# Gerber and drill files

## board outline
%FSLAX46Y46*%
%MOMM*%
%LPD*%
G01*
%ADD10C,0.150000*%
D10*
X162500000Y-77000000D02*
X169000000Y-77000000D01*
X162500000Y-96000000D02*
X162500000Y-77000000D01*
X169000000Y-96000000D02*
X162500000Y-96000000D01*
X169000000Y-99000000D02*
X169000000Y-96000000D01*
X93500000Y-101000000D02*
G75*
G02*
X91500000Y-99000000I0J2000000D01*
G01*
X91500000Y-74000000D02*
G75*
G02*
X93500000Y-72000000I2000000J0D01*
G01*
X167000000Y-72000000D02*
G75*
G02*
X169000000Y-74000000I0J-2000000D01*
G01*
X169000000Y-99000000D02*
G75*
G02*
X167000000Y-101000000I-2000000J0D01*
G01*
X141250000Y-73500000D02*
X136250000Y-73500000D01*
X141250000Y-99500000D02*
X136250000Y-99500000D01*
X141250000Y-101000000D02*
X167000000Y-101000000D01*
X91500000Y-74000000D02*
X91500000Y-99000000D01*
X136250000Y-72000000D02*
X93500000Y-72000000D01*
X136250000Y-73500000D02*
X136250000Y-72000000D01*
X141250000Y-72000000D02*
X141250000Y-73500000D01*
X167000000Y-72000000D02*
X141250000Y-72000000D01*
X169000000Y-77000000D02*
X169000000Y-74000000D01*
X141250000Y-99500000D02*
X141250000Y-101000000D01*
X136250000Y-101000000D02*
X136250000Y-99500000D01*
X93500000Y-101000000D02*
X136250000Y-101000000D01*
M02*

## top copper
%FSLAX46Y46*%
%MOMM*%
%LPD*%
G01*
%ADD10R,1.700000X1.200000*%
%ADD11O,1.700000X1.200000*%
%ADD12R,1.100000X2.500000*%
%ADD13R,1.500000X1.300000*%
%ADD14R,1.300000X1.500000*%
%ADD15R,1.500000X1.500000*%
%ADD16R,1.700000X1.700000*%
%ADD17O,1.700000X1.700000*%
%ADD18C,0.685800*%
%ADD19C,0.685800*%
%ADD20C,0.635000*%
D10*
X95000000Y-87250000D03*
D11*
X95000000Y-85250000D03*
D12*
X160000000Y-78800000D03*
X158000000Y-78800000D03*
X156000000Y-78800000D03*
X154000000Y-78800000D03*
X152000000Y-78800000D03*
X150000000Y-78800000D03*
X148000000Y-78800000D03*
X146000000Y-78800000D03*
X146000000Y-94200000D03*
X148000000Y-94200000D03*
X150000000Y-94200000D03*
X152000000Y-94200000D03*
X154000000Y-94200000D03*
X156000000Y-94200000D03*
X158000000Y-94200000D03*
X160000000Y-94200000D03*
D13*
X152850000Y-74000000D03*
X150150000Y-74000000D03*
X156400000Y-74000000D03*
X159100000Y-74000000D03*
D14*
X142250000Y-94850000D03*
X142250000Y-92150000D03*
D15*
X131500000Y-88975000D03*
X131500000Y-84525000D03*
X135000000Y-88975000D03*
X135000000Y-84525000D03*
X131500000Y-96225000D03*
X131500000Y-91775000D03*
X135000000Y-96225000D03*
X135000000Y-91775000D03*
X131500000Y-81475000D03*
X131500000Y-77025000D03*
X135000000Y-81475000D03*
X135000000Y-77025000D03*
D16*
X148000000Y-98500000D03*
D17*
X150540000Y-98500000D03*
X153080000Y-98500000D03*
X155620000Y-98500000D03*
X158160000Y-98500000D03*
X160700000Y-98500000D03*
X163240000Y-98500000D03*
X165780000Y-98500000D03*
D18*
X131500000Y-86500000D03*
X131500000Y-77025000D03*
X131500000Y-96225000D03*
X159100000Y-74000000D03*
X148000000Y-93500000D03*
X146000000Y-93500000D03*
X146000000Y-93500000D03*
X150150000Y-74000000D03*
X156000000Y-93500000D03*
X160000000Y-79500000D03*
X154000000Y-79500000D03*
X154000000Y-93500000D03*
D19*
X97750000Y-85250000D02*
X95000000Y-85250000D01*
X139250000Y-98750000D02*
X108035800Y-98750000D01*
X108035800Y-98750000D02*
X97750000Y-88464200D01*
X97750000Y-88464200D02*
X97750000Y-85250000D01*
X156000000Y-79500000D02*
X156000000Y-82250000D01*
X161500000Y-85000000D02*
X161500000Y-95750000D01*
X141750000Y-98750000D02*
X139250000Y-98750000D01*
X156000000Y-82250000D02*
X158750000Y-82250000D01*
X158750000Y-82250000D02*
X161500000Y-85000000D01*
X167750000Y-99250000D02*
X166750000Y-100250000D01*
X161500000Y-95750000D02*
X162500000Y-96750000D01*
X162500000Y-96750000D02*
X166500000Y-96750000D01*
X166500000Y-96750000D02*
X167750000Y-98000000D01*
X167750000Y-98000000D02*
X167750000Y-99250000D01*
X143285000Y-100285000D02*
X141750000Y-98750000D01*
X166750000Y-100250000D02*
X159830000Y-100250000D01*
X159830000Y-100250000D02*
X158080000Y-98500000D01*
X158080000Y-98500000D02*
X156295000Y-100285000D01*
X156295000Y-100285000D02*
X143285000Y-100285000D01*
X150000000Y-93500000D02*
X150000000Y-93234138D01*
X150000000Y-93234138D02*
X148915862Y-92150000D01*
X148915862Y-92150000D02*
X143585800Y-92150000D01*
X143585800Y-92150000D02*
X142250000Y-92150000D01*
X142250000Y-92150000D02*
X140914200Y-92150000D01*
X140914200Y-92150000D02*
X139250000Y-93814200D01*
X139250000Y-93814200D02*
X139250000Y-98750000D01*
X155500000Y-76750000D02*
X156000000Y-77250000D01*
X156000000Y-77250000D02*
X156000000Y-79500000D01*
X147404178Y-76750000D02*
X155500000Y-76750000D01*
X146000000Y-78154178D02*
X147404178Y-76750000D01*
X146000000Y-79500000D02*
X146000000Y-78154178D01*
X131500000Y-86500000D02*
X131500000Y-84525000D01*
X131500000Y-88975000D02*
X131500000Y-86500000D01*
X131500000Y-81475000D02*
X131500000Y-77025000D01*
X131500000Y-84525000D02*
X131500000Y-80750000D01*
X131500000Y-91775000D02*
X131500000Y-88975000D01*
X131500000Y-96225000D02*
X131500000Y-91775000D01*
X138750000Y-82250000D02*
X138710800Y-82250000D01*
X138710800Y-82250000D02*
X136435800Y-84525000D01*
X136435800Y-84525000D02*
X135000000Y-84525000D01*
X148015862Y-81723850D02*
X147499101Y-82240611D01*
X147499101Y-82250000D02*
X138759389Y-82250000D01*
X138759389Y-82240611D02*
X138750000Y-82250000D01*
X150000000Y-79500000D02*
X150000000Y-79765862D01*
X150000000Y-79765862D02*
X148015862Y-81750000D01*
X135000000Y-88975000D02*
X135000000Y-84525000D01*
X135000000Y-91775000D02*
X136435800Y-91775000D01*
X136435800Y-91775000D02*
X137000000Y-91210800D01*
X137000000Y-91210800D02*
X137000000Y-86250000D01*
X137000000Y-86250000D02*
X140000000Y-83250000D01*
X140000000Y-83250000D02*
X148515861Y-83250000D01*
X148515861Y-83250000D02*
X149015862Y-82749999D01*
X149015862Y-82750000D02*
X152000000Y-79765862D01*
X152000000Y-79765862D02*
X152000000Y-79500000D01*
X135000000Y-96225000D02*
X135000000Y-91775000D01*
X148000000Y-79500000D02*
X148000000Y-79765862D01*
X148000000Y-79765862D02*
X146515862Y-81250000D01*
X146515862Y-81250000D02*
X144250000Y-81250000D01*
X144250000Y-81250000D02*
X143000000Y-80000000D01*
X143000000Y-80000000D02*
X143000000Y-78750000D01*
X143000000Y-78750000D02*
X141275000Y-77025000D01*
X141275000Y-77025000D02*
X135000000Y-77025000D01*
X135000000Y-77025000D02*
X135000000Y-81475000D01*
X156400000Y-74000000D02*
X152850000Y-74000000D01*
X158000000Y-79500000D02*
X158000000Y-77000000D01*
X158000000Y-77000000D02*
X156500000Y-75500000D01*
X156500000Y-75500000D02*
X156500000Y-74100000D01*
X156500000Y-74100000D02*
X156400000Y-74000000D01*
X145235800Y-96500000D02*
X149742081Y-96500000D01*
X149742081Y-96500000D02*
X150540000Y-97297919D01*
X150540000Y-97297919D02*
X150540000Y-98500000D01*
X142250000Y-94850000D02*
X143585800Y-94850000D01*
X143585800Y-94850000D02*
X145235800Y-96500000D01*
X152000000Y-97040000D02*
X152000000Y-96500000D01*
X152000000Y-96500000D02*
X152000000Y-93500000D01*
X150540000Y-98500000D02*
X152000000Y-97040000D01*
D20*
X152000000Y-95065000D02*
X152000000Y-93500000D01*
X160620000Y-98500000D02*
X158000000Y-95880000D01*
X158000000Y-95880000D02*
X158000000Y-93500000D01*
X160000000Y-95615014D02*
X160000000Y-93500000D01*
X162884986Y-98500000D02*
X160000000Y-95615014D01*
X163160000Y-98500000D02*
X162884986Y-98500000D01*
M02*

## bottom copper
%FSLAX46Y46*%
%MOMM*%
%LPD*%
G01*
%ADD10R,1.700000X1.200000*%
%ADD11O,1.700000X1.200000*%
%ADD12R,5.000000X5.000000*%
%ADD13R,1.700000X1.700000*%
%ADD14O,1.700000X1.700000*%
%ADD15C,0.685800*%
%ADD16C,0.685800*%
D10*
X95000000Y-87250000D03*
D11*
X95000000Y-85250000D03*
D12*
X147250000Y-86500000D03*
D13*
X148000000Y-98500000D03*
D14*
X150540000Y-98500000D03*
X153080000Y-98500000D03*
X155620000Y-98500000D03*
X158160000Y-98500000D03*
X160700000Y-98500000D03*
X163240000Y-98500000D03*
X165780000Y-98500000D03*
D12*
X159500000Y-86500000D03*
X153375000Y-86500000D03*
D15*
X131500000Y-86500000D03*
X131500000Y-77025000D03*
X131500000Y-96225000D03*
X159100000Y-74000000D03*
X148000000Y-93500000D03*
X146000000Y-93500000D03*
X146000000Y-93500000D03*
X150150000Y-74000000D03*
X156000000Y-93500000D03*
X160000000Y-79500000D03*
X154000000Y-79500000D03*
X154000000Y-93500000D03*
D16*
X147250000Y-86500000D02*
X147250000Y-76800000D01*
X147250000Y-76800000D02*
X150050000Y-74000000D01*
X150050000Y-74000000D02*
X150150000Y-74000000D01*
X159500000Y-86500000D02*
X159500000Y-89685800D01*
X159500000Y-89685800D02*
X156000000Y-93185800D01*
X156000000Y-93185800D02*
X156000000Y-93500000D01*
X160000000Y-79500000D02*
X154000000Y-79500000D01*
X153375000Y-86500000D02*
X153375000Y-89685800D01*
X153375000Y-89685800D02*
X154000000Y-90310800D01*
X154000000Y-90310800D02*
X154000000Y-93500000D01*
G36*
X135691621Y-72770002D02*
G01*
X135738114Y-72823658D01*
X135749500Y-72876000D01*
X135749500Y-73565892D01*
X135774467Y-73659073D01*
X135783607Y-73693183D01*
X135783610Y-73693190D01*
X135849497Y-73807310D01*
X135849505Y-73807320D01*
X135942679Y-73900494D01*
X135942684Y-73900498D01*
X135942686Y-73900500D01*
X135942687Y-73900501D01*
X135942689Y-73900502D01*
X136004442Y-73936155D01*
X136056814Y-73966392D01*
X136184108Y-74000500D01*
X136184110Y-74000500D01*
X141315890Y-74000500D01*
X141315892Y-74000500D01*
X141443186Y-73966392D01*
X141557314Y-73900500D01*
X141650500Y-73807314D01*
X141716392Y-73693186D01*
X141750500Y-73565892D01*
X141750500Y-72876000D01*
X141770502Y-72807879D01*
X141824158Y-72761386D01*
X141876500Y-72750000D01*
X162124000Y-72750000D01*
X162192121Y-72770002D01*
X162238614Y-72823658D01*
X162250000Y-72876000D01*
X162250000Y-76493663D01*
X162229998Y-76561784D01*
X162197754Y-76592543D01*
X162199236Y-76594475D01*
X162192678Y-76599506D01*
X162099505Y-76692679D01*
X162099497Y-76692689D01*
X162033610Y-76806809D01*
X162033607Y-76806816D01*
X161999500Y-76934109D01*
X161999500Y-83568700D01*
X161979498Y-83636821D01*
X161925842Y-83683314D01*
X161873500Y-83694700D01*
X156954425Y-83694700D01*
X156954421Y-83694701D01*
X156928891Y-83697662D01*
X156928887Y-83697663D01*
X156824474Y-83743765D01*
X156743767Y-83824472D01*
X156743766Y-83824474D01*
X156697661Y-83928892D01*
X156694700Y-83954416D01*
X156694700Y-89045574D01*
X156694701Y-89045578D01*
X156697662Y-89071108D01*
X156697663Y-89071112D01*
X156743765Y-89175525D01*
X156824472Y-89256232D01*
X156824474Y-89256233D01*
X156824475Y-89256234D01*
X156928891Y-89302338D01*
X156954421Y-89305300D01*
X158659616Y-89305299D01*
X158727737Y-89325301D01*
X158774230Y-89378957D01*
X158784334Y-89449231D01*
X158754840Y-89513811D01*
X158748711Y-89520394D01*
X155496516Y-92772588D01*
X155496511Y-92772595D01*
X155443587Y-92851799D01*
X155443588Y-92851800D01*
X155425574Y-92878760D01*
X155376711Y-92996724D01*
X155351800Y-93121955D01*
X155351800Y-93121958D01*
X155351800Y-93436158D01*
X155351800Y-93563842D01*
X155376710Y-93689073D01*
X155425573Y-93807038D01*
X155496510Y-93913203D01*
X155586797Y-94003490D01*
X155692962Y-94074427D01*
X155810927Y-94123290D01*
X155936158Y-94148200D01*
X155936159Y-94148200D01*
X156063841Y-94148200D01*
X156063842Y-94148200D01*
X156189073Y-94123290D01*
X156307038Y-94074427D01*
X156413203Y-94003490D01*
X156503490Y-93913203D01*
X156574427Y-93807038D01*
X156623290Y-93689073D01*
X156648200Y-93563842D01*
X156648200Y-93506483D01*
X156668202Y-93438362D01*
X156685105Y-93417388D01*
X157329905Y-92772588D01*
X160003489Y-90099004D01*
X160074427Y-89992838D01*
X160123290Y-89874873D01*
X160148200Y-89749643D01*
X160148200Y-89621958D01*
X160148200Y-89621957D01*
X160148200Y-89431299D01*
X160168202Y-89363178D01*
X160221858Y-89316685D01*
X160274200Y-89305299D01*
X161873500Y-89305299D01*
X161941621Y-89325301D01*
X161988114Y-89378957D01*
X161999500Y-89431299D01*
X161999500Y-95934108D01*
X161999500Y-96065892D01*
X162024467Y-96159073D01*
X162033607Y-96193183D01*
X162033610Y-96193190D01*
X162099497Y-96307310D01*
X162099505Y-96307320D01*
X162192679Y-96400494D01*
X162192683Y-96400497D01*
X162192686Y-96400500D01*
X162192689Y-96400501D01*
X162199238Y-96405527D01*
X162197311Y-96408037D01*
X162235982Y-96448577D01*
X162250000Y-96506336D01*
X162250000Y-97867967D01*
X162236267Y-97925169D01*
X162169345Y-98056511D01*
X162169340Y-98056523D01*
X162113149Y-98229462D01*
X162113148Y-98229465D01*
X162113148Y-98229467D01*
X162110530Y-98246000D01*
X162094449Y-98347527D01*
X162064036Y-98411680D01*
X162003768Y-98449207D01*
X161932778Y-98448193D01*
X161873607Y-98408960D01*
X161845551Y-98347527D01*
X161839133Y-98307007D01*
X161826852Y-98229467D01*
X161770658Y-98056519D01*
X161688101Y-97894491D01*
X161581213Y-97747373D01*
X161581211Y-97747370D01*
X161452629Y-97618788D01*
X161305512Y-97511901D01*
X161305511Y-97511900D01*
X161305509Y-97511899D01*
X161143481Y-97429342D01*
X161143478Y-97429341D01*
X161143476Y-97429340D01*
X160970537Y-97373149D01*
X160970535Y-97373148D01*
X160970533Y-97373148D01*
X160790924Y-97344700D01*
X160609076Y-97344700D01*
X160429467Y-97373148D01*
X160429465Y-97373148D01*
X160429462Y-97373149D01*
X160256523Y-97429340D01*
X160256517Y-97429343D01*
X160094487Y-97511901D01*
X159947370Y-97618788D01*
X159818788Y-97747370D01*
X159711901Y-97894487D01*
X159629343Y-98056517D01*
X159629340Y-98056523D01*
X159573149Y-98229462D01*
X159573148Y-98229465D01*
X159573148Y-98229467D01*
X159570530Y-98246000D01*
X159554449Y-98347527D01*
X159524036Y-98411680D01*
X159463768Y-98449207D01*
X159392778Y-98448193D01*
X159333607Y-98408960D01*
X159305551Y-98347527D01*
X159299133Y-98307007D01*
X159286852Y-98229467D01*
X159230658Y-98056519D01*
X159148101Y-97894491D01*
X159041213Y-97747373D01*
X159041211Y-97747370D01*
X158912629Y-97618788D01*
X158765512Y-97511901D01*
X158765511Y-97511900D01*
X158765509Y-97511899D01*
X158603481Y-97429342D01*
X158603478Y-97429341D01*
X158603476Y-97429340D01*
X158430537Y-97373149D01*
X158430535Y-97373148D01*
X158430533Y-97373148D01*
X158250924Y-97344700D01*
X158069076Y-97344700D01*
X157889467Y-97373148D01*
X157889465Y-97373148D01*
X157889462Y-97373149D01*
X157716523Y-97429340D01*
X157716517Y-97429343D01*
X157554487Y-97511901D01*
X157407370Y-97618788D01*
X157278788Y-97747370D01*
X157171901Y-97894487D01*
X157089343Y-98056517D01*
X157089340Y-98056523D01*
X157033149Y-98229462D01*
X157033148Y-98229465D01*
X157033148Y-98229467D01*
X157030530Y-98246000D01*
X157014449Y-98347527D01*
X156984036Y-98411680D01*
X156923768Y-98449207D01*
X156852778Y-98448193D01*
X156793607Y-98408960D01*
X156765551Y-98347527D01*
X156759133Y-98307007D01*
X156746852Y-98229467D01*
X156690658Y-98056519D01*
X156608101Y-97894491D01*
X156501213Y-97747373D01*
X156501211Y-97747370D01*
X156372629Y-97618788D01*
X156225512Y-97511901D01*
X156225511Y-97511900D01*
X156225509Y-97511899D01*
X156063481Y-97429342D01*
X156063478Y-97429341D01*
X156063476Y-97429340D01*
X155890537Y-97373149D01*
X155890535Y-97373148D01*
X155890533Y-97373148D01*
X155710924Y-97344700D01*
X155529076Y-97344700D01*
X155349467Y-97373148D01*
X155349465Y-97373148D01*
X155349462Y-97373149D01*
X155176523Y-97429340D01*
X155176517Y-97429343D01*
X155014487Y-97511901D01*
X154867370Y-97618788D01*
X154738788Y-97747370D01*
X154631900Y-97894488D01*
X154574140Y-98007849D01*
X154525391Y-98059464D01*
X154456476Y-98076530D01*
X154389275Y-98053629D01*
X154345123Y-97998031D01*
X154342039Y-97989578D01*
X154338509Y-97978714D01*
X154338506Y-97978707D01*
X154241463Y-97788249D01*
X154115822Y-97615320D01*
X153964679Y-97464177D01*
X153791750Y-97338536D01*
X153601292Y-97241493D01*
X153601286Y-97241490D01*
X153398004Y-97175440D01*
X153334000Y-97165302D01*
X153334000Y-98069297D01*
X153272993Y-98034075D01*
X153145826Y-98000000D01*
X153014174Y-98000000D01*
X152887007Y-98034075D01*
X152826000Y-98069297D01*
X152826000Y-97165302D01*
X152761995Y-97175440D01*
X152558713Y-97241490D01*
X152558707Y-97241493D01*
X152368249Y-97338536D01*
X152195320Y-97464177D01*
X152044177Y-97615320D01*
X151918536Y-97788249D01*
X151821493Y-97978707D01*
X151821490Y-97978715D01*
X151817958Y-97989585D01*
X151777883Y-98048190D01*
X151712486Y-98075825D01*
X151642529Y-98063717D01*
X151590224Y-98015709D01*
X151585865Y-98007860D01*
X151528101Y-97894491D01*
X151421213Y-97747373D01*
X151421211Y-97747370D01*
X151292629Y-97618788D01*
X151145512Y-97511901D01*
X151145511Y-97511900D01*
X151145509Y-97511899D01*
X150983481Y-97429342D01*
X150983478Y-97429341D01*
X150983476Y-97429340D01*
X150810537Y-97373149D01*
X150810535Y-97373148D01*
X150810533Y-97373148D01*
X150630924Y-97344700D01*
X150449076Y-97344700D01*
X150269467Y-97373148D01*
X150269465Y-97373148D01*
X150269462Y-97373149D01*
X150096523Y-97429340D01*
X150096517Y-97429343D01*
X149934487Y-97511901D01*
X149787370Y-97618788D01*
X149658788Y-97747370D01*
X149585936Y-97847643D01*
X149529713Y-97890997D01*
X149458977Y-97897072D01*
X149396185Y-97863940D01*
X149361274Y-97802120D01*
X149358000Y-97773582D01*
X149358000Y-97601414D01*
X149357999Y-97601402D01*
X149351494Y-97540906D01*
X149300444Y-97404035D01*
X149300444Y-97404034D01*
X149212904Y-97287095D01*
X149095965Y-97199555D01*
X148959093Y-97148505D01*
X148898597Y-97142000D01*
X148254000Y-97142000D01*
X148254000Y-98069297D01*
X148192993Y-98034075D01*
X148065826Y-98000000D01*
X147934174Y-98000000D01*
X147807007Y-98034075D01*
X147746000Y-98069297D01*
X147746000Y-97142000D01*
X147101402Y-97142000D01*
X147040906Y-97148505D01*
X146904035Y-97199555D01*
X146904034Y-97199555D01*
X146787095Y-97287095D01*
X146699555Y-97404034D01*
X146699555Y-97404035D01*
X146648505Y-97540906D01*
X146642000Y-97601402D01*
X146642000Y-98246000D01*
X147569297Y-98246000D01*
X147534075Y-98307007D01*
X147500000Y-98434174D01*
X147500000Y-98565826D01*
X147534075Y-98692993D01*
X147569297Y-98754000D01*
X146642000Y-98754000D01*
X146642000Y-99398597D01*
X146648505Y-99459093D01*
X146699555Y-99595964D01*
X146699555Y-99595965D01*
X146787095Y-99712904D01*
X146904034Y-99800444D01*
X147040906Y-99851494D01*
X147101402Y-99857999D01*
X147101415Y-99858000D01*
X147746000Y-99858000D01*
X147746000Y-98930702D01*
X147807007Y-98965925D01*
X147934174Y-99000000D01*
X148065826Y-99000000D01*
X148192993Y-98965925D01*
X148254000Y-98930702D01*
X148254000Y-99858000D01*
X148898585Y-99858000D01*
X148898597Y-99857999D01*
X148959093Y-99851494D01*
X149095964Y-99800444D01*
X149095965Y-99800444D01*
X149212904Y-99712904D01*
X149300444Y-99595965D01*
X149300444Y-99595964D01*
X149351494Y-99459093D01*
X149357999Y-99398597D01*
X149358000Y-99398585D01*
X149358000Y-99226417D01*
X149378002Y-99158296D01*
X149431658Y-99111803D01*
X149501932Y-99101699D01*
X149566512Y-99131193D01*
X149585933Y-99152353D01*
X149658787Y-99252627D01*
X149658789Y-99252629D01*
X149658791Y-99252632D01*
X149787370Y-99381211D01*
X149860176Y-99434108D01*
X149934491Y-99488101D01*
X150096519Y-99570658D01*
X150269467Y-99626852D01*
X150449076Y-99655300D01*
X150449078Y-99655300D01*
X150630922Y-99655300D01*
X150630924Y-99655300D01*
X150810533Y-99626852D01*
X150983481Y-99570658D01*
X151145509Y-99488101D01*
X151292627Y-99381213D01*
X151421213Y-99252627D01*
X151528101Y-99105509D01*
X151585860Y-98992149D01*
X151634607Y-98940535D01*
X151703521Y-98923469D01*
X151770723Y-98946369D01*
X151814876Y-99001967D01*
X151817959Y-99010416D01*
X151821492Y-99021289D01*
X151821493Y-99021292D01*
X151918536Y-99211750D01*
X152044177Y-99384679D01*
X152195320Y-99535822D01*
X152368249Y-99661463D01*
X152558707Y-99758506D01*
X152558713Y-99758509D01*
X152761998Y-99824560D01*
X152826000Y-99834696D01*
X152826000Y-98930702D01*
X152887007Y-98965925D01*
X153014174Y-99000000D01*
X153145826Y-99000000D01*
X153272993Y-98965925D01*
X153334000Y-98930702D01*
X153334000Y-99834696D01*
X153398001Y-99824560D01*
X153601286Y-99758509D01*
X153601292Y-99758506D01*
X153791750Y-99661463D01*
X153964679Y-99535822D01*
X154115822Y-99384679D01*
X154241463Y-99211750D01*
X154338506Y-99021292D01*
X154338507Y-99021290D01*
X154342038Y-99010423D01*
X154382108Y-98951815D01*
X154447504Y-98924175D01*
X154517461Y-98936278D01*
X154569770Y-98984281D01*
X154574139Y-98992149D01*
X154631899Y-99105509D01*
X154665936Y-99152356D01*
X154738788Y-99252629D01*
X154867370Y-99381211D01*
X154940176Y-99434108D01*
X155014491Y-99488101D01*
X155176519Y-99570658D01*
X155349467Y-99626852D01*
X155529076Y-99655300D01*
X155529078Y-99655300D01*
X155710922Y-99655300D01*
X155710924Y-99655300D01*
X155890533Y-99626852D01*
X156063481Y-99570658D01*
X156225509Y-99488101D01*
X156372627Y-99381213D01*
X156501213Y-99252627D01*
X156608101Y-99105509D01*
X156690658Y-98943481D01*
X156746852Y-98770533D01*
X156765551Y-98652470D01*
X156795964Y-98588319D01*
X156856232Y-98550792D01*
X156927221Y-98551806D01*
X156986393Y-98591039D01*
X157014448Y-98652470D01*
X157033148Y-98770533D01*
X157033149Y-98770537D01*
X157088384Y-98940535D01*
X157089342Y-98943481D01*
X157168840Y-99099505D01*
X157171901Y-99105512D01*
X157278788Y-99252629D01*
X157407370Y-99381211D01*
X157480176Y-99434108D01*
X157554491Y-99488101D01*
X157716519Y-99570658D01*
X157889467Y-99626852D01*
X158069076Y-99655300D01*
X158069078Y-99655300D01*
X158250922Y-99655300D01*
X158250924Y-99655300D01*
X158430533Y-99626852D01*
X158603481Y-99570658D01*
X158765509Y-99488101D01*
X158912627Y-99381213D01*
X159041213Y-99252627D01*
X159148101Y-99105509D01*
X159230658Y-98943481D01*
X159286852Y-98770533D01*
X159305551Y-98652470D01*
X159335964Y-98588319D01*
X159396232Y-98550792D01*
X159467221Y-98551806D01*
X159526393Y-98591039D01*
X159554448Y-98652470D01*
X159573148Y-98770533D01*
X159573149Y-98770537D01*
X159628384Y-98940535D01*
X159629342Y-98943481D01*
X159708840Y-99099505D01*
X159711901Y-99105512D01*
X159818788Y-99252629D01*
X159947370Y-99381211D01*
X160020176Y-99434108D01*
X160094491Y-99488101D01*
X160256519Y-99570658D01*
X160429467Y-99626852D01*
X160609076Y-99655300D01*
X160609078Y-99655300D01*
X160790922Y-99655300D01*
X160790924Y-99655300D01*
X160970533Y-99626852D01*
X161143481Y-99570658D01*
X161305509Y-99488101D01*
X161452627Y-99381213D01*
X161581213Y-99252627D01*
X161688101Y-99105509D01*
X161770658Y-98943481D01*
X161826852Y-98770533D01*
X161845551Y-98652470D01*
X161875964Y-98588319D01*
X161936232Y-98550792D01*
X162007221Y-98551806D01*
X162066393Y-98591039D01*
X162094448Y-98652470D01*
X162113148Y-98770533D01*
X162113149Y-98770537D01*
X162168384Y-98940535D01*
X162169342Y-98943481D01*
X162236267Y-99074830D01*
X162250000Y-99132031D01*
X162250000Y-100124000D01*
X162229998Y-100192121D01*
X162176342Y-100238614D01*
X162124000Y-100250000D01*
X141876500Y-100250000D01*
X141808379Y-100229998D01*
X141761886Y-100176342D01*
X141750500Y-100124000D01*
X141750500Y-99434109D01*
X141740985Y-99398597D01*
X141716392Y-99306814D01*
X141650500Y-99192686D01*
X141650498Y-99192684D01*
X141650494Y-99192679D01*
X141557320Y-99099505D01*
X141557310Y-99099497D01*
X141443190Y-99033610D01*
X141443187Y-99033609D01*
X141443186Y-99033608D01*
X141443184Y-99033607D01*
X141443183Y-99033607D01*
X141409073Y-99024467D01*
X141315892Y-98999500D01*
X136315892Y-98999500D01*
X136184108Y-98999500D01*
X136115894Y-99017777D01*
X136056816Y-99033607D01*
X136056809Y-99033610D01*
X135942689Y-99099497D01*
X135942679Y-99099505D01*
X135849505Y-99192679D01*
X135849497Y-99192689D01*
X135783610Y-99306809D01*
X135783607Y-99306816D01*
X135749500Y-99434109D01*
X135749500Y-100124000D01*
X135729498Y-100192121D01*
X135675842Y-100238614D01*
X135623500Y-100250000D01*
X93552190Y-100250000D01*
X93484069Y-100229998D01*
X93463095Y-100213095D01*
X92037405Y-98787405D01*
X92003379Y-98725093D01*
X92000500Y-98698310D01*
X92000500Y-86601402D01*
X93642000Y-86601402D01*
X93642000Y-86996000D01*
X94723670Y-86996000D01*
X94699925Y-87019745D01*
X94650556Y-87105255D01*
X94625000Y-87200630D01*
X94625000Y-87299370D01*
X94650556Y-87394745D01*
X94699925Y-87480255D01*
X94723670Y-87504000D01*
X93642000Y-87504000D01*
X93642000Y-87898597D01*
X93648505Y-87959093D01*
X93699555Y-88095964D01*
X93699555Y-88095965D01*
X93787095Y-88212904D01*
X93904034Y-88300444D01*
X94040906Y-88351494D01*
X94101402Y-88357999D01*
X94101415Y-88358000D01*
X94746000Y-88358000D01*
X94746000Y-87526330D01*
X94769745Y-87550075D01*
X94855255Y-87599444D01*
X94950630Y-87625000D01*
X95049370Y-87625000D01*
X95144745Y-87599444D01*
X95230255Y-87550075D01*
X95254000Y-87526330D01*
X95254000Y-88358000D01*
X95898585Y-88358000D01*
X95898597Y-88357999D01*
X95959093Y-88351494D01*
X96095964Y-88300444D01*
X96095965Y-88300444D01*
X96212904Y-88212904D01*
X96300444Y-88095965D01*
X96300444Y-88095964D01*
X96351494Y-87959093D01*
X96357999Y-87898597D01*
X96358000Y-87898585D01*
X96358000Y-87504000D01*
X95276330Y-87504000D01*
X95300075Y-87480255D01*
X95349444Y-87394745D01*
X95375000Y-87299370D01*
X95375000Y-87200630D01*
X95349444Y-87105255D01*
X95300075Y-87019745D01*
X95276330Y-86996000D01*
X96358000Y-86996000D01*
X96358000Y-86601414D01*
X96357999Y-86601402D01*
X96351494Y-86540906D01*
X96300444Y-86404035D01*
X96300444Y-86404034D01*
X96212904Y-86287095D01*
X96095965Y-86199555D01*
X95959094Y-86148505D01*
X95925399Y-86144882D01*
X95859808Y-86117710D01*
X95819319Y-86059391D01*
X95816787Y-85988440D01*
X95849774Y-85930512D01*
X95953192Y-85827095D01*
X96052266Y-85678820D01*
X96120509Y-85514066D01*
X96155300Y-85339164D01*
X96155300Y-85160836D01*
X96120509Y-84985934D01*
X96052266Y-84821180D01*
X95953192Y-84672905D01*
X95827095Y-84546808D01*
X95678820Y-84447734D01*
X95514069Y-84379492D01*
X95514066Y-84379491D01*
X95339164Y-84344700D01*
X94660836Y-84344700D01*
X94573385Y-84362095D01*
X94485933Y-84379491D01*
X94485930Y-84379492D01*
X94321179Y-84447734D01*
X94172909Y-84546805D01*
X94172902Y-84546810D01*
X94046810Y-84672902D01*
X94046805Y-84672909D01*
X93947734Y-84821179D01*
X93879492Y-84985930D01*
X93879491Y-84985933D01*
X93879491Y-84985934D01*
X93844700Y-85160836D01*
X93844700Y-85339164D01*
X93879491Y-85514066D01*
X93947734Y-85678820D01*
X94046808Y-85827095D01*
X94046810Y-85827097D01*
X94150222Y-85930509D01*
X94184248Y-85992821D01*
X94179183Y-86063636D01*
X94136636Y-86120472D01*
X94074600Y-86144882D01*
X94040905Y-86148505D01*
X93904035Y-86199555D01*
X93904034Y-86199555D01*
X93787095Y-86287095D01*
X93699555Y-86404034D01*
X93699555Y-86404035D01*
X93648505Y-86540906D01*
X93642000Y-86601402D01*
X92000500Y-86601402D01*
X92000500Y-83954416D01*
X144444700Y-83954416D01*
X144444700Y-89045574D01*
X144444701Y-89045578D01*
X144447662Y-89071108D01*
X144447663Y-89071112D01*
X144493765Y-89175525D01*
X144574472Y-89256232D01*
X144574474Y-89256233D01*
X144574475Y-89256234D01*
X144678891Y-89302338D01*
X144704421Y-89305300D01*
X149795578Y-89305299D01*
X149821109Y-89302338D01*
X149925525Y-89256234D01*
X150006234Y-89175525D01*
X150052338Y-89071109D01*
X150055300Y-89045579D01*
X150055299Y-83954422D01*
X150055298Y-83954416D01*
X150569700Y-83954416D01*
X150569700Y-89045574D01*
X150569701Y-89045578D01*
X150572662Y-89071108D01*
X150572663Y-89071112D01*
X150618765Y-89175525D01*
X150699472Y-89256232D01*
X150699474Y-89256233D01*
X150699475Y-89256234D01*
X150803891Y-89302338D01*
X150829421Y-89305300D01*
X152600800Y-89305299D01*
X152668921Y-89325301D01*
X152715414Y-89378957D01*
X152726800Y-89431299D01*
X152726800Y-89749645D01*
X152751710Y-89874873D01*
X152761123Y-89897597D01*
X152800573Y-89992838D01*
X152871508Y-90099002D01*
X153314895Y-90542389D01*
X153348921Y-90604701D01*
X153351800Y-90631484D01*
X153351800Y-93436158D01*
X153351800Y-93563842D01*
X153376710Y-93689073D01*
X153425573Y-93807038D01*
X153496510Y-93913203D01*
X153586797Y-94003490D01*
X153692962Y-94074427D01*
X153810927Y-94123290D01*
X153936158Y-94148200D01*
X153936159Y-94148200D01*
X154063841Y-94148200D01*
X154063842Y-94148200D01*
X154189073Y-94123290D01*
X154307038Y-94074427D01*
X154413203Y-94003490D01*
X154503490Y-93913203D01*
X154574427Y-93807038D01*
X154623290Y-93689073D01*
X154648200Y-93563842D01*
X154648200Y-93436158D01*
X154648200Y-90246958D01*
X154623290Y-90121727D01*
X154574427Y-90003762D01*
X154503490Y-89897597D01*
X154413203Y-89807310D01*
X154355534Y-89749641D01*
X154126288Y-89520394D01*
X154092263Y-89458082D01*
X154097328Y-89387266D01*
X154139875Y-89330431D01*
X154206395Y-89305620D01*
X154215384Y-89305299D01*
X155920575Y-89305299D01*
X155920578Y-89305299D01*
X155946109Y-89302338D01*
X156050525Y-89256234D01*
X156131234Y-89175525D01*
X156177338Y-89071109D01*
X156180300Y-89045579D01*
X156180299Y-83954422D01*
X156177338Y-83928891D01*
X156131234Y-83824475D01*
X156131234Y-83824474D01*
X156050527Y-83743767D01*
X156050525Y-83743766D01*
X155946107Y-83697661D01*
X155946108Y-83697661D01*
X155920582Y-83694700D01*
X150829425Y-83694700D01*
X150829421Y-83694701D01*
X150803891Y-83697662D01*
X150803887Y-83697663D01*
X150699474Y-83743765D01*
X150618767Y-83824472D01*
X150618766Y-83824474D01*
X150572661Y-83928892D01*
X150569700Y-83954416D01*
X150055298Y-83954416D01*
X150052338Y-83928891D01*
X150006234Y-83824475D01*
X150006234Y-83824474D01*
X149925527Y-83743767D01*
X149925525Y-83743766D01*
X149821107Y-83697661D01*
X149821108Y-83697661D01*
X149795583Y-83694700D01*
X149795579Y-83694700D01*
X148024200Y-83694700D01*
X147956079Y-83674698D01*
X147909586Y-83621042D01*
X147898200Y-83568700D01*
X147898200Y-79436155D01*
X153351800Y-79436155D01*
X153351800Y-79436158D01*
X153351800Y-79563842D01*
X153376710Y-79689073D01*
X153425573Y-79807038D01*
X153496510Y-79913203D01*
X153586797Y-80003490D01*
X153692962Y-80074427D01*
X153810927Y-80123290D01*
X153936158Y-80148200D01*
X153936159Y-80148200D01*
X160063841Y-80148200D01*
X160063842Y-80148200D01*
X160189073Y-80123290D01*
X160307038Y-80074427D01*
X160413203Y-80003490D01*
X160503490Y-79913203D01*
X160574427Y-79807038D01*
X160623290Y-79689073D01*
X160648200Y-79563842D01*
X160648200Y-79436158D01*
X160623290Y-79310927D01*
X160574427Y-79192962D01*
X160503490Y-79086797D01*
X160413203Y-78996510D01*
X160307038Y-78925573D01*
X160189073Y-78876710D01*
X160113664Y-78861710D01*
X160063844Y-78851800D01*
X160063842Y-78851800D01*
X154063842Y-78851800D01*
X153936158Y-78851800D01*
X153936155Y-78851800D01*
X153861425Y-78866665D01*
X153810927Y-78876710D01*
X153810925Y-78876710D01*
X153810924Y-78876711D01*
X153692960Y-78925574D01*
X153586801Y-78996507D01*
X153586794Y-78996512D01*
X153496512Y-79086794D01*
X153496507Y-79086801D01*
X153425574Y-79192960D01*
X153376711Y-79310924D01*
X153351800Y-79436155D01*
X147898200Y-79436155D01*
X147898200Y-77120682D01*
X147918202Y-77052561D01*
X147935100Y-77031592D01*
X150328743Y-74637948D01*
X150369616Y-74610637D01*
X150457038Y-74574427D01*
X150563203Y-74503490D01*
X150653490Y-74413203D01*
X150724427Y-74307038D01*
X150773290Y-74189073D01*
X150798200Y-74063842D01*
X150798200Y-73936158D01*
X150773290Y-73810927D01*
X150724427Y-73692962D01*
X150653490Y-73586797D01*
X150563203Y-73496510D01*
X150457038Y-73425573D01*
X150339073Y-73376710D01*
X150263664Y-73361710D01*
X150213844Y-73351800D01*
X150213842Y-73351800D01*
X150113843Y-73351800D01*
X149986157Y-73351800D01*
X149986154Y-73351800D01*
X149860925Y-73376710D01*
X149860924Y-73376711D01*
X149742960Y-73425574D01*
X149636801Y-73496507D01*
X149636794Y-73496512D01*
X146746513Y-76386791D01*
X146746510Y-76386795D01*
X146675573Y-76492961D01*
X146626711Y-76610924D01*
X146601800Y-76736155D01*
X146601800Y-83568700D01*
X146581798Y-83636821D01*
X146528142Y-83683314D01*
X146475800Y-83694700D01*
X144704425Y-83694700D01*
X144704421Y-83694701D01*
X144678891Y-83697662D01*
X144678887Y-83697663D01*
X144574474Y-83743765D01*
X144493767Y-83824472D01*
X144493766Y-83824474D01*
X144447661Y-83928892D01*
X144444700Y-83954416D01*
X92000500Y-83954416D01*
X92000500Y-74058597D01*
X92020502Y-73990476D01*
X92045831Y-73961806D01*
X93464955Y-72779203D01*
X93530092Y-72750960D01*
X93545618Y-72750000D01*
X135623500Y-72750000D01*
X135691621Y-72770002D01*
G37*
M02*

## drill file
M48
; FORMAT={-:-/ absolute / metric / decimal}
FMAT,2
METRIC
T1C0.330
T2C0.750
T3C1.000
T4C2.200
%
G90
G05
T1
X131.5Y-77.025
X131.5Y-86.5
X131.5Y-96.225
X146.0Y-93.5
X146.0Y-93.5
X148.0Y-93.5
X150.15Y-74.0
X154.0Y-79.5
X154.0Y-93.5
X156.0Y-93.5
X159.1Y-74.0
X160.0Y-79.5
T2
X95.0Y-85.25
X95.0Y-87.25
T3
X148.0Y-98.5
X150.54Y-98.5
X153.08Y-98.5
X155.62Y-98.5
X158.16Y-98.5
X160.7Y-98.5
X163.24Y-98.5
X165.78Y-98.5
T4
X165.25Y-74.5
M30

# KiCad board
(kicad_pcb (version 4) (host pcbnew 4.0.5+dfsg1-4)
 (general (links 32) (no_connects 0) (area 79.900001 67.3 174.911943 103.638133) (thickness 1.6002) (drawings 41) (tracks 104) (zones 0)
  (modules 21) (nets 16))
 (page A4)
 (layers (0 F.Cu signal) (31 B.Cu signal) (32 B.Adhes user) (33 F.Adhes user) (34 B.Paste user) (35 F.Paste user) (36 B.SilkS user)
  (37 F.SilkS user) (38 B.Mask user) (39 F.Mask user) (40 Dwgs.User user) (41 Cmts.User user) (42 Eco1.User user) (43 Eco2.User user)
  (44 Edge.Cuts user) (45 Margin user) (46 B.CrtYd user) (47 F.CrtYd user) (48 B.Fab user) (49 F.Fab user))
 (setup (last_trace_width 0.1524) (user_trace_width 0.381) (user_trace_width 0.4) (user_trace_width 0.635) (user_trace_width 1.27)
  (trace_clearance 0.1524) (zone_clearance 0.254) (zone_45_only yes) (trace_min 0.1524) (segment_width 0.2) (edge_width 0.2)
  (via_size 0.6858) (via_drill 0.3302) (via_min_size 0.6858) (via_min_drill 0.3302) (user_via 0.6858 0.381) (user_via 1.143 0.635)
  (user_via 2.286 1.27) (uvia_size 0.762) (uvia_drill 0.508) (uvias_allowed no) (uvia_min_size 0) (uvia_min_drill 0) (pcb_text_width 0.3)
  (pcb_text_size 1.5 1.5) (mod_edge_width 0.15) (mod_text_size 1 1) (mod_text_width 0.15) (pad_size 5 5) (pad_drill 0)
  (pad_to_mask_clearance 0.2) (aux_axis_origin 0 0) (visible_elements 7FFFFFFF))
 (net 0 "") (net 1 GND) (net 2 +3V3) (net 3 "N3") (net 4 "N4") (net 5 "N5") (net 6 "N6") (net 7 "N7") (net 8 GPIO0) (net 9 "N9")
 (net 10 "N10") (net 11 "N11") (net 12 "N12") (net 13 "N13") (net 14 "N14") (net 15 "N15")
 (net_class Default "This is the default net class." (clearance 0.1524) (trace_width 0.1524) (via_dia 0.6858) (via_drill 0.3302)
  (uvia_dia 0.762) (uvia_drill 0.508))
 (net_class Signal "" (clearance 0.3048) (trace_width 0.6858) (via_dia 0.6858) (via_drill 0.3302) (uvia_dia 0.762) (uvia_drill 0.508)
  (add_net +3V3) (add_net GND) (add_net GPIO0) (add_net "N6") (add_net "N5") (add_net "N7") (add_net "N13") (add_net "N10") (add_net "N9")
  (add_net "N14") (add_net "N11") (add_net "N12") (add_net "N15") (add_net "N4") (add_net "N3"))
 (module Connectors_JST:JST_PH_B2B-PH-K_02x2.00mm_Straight (layer B.Cu) (at 95 87.25 90)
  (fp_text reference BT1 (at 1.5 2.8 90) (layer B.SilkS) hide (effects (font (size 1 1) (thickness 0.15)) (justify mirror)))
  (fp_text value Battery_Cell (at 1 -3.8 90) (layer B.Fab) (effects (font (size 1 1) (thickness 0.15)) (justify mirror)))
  (pad 2 thru_hole rect (at 0 0 90) (size 1.2 1.7) (drill 0.75) (layers *.Cu *.Mask) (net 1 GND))
  (pad 1 thru_hole oval (at 2 0 90) (size 1.2 1.7) (drill 0.75) (layers *.Cu *.Mask) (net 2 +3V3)))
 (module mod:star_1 (layer F.Cu) (at 129.5 96.25 270)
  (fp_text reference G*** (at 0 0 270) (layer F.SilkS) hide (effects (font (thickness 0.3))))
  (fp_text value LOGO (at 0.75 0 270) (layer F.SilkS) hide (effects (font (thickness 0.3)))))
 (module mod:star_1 (layer F.Cu) (at 129.5 91.75 270)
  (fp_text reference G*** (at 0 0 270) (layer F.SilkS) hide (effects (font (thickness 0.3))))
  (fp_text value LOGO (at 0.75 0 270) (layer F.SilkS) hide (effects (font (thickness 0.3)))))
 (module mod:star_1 (layer F.Cu) (at 129.5 94 270)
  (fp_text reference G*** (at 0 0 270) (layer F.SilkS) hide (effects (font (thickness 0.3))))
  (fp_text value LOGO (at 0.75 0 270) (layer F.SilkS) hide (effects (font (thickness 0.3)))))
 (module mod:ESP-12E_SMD (layer F.Cu) (at 160 79.5 270)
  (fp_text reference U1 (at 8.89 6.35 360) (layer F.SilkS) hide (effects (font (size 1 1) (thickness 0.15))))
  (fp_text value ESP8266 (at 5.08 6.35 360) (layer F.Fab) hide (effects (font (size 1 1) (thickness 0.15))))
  (pad 1 smd rect (at 0 0 270) (size 2.5 1.1) (drill (offset -0.7 0)) (layers F.Cu F.Paste F.Mask) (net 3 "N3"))
  (pad 2 smd rect (at 0 2 270) (size 2.5 1.1) (drill (offset -0.7 0)) (layers F.Cu F.Paste F.Mask) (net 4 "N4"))
  (pad 3 smd rect (at 0 4 270) (size 2.5 1.1) (drill (offset -0.7 0)) (layers F.Cu F.Paste F.Mask) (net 2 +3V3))
  (pad 4 smd rect (at 0 6 270) (size 2.5 1.1) (drill (offset -0.7 0)) (layers F.Cu F.Paste F.Mask) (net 3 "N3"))
  (pad 5 smd rect (at 0 8 270) (size 2.5 1.1) (drill (offset -0.7 0)) (layers F.Cu F.Paste F.Mask) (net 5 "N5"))
  (pad 6 smd rect (at 0 10 270) (size 2.5 1.1) (drill (offset -0.7 0)) (layers F.Cu F.Paste F.Mask) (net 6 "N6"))
  (pad 7 smd rect (at 0 12 270) (size 2.5 1.1) (drill (offset -0.7 0)) (layers F.Cu F.Paste F.Mask) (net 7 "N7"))
  (pad 8 smd rect (at 0 14 270) (size 2.5 1.1) (drill (offset -0.7 0)) (layers F.Cu F.Paste F.Mask) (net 2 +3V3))
  (pad 9 smd rect (at 14 14 270) (size 2.5 1.1) (drill (offset 0.7 0)) (layers F.Cu F.Paste F.Mask) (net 1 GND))
  (pad 10 smd rect (at 14 12 270) (size 2.5 1.1) (drill (offset 0.7 0)) (layers F.Cu F.Paste F.Mask) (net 1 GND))
  (pad 11 smd rect (at 14 10 270) (size 2.5 1.1) (drill (offset 0.7 0)) (layers F.Cu F.Paste F.Mask) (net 2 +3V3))
  (pad 12 smd rect (at 14 8 270) (size 2.5 1.1) (drill (offset 0.7 0)) (layers F.Cu F.Paste F.Mask) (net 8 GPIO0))
  (pad 13 smd rect (at 14 6 270) (size 2.5 1.1) (drill (offset 0.7 0)) (layers F.Cu F.Paste F.Mask) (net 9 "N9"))
  (pad 14 smd rect (at 14 4 270) (size 2.5 1.1) (drill (offset 0.7 0)) (layers F.Cu F.Paste F.Mask) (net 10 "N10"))
  (pad 15 smd rect (at 14 2 270) (size 2.5 1.1) (drill (offset 0.7 0)) (layers F.Cu F.Paste F.Mask) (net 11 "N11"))
  (pad 16 smd rect (at 14 0 270) (size 2.5 1.1) (drill (offset 0.7 0)) (layers F.Cu F.Paste F.Mask) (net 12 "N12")))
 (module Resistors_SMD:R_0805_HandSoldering (layer F.Cu) (at 151.5 74 180)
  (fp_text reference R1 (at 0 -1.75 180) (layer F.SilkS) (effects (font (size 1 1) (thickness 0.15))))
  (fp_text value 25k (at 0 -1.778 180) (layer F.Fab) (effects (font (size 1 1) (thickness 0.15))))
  (pad 1 smd rect (at -1.35 0 180) (size 1.5 1.3) (layers F.Cu F.Paste F.Mask) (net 4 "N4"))
  (pad 2 smd rect (at 1.35 0 180) (size 1.5 1.3) (layers F.Cu F.Paste F.Mask) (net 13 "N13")))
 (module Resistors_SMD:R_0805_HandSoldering (layer F.Cu) (at 157.75 74)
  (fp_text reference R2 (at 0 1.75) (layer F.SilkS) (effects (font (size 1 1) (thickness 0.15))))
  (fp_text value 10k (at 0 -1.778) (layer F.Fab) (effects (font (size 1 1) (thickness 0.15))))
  (pad 1 smd rect (at -1.35 0) (size 1.5 1.3) (layers F.Cu F.Paste F.Mask) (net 4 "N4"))
  (pad 2 smd rect (at 1.35 0) (size 1.5 1.3) (layers F.Cu F.Paste F.Mask) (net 1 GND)))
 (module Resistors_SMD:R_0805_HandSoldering (layer F.Cu) (at 142.25 93.5 90)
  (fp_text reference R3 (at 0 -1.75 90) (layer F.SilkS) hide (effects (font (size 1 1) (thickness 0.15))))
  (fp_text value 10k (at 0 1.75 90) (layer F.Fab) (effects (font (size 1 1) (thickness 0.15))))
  (pad 1 smd rect (at -1.35 0 90) (size 1.5 1.3) (layers F.Cu F.Paste F.Mask) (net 8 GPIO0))
  (pad 2 smd rect (at 1.35 0 90) (size 1.5 1.3) (layers F.Cu F.Paste F.Mask) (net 2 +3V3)))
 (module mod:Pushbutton (layer F.Cu) (at 133.25 86.75 90)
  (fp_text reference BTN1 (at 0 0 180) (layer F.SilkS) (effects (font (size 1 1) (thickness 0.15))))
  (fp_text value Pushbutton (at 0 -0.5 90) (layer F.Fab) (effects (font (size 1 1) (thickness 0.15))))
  (pad 1 smd rect (at -2.225 -1.75 90) (size 1.5 1.5) (layers F.Cu F.Paste F.Mask) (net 1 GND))
  (pad 1 smd rect (at 2.225 -1.75 90) (size 1.5 1.5) (layers F.Cu F.Paste F.Mask) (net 1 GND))
  (pad 2 smd rect (at -2.225 1.75 90) (size 1.5 1.5) (layers F.Cu F.Paste F.Mask) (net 6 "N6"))
  (pad 2 smd rect (at 2.225 1.75 90) (size 1.5 1.5) (layers F.Cu F.Paste F.Mask) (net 6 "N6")))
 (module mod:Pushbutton (layer F.Cu) (at 133.25 94 90)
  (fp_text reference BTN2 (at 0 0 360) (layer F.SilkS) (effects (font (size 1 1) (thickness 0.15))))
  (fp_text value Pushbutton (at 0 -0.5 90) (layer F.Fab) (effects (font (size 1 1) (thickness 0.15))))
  (pad 1 smd rect (at -2.225 -1.75 90) (size 1.5 1.5) (layers F.Cu F.Paste F.Mask) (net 1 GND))
  (pad 1 smd rect (at 2.225 -1.75 90) (size 1.5 1.5) (layers F.Cu F.Paste F.Mask) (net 1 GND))
  (pad 2 smd rect (at -2.225 1.75 90) (size 1.5 1.5) (layers F.Cu F.Paste F.Mask) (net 5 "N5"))
  (pad 2 smd rect (at 2.225 1.75 90) (size 1.5 1.5) (layers F.Cu F.Paste F.Mask) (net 5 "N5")))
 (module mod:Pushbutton (layer F.Cu) (at 133.25 79.25 90)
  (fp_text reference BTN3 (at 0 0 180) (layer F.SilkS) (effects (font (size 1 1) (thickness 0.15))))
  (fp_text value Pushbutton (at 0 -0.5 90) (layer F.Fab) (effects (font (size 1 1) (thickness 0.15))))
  (pad 1 smd rect (at -2.225 -1.75 90) (size 1.5 1.5) (layers F.Cu F.Paste F.Mask) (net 1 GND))
  (pad 1 smd rect (at 2.225 -1.75 90) (size 1.5 1.5) (layers F.Cu F.Paste F.Mask) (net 1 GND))
  (pad 2 smd rect (at -2.225 1.75 90) (size 1.5 1.5) (layers F.Cu F.Paste F.Mask) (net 7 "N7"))
  (pad 2 smd rect (at 2.225 1.75 90) (size 1.5 1.5) (layers F.Cu F.Paste F.Mask) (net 7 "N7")))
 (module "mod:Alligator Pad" (layer B.Cu) (at 147.25 86.5)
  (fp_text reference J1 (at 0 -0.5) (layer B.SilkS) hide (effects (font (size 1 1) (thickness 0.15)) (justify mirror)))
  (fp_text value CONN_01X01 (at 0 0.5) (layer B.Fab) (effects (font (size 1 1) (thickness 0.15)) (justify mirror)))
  (pad 1 smd rect (at 0 0) (size 5 5) (layers B.Cu B.Mask) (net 13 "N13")))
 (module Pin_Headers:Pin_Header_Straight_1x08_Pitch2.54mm (layer F.Cu) (at 148 98.5 90)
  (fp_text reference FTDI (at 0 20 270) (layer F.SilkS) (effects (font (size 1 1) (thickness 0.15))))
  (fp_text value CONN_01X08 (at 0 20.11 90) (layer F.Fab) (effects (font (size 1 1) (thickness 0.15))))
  (pad 1 thru_hole rect (at 0 0 90) (size 1.7 1.7) (drill 1) (layers *.Cu *.Mask) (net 1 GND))
  (pad 2 thru_hole oval (at 0 2.54 90) (size 1.7 1.7) (drill 1) (layers *.Cu *.Mask) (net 8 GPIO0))
  (pad 3 thru_hole oval (at 0 5.08 90) (size 1.7 1.7) (drill 1) (layers *.Cu *.Mask) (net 1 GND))
  (pad 4 thru_hole oval (at 0 7.62 90) (size 1.7 1.7) (drill 1) (layers *.Cu *.Mask) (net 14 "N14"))
  (pad 5 thru_hole oval (at 0 10.16 90) (size 1.7 1.7) (drill 1) (layers *.Cu *.Mask) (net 2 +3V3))
  (pad 6 thru_hole oval (at 0 12.7 90) (size 1.7 1.7) (drill 1) (layers *.Cu *.Mask) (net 11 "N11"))
  (pad 7 thru_hole oval (at 0 15.24 90) (size 1.7 1.7) (drill 1) (layers *.Cu *.Mask) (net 12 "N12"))
  (pad 8 thru_hole oval (at 0 17.78 90) (size 1.7 1.7) (drill 1) (layers *.Cu *.Mask) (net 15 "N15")))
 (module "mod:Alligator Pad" (layer B.Cu) (at 159.5 86.5)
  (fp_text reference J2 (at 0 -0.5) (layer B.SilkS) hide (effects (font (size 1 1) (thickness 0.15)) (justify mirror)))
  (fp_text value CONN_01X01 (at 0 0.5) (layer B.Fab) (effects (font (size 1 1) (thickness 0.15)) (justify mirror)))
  (pad 1 smd rect (at 0 0) (size 5 5) (layers B.Cu B.Mask) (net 10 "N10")))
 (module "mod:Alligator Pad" (layer B.Cu) (at 153.5 86.5)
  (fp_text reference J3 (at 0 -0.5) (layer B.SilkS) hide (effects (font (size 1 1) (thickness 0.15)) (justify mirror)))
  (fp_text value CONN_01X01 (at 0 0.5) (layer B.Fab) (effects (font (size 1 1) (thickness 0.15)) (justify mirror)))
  (pad 1 smd rect (at -0.125 0) (size 5 5) (layers B.Cu B.Mask) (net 9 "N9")))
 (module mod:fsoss (layer F.Cu) (at 105 86.25 270)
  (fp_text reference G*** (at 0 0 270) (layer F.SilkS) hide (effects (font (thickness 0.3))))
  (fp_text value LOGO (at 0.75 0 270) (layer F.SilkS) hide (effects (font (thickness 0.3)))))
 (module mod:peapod (layer F.Cu) (at 112.75 86 270)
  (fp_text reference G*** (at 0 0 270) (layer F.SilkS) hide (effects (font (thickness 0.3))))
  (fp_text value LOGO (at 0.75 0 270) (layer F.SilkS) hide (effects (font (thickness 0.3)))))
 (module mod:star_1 (layer F.Cu) (at 129.5 79.25 270)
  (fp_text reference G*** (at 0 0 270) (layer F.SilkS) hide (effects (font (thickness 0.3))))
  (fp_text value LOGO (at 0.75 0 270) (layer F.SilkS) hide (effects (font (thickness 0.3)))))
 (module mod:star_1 (layer F.Cu) (at 129.5 85.5 270)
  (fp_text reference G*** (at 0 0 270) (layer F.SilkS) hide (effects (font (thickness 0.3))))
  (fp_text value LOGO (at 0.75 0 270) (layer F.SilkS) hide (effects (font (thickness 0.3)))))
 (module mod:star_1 (layer F.Cu) (at 129.5 88 270)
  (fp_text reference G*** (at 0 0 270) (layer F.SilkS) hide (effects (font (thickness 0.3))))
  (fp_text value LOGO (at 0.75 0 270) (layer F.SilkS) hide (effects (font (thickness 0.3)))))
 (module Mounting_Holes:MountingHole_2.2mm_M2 (layer F.Cu) (at 165.25 74.5)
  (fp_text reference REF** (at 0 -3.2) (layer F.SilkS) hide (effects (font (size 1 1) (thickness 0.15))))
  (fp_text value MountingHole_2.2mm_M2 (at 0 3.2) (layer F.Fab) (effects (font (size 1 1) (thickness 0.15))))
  (pad 1 np_thru_hole circle (at 0 0) (size 2.2 2.2) (drill 2.2) (layers *.Cu *.Mask)))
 (gr_line (start 162.5 77) (end 169 77) (angle 90) (layer Edge.Cuts) (width 0.15))
 (gr_line (start 162.5 96) (end 162.5 77) (angle 90) (layer Edge.Cuts) (width 0.15))
 (gr_line (start 169 96) (end 162.5 96) (angle 90) (layer Edge.Cuts) (width 0.15))
 (gr_line (start 169 99) (end 169 96) (angle 90) (layer Edge.Cuts) (width 0.15))
 (gr_arc (start 93.5 99) (end 93.5 101) (angle 90) (layer Edge.Cuts) (width 0.15))
 (gr_arc (start 93.5 74) (end 91.5 74) (angle 90) (layer Edge.Cuts) (width 0.15))
 (gr_arc (start 167 74) (end 167 72) (angle 90) (layer Edge.Cuts) (width 0.15))
 (gr_arc (start 167 99) (end 169 99) (angle 90) (layer Edge.Cuts) (width 0.15))
 (gr_line (start 141.25 73.5) (end 136.25 73.5) (angle 90) (layer Edge.Cuts) (width 0.15))
 (gr_line (start 141.25 99.5) (end 136.25 99.5) (angle 90) (layer Edge.Cuts) (width 0.15))
 (gr_line (start 141.25 101) (end 167 101) (angle 90) (layer Edge.Cuts) (width 0.15))
 (gr_line (start 91.5 74) (end 91.5 99) (angle 90) (layer Edge.Cuts) (width 0.15))
 (gr_line (start 136.25 72) (end 93.5 72) (angle 90) (layer Edge.Cuts) (width 0.15))
 (gr_line (start 136.25 73.5) (end 136.25 72) (angle 90) (layer Edge.Cuts) (width 0.15))
 (gr_line (start 141.25 72) (end 141.25 73.5) (angle 90) (layer Edge.Cuts) (width 0.15))
 (gr_line (start 167 72) (end 141.25 72) (angle 90) (layer Edge.Cuts) (width 0.15))
 (gr_line (start 169 77) (end 169 74) (angle 90) (layer Edge.Cuts) (width 0.15))
 (gr_line (start 141.25 99.5) (end 141.25 101) (angle 90) (layer Edge.Cuts) (width 0.15))
 (gr_line (start 136.25 101) (end 136.25 99.5) (angle 90) (layer Edge.Cuts) (width 0.15))
 (gr_line (start 93.5 101) (end 136.25 101) (angle 90) (layer Edge.Cuts) (width 0.15))
 (segment (start 97.75 85.25) (end 95 85.25) (width 0.6858) (layer F.Cu) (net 2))
 (segment (start 139.25 98.75) (end 108.0358 98.75) (width 0.6858) (layer F.Cu) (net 2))
 (segment (start 108.0358 98.75) (end 97.75 88.4642) (width 0.6858) (layer F.Cu) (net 2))
 (segment (start 97.75 88.4642) (end 97.75 85.25) (width 0.6858) (layer F.Cu) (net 2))
 (segment (start 156 79.5) (end 156 82.25) (width 0.6858) (layer F.Cu) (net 2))
 (segment (start 161.5 85) (end 161.5 95.75) (width 0.6858) (layer F.Cu) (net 2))
 (segment (start 141.75 98.75) (end 139.25 98.75) (width 0.6858) (layer F.Cu) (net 2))
 (segment (start 156 82.25) (end 158.75 82.25) (width 0.6858) (layer F.Cu) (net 2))
 (segment (start 158.75 82.25) (end 161.5 85) (width 0.6858) (layer F.Cu) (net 2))
 (segment (start 167.75 99.25) (end 166.75 100.25) (width 0.6858) (layer F.Cu) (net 2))
 (segment (start 161.5 95.75) (end 162.5 96.75) (width 0.6858) (layer F.Cu) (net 2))
 (segment (start 162.5 96.75) (end 166.5 96.75) (width 0.6858) (layer F.Cu) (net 2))
 (segment (start 166.5 96.75) (end 167.75 98) (width 0.6858) (layer F.Cu) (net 2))
 (segment (start 167.75 98) (end 167.75 99.25) (width 0.6858) (layer F.Cu) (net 2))
 (segment (start 143.285 100.285) (end 141.75 98.75) (width 0.6858) (layer F.Cu) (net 2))
 (segment (start 166.75 100.25) (end 159.83 100.25) (width 0.6858) (layer F.Cu) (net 2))
 (segment (start 159.83 100.25) (end 158.08 98.5) (width 0.6858) (layer F.Cu) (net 2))
 (segment (start 158.08 98.5) (end 156.295 100.285) (width 0.6858) (layer F.Cu) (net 2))
 (segment (start 156.295 100.285) (end 143.285 100.285) (width 0.6858) (layer F.Cu) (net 2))
 (segment (start 150 93.5) (end 150 93.234138) (width 0.6858) (layer F.Cu) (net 2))
 (segment (start 150 93.234138) (end 148.915862 92.15) (width 0.6858) (layer F.Cu) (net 2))
 (segment (start 148.915862 92.15) (end 143.5858 92.15) (width 0.6858) (layer F.Cu) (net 2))
 (segment (start 143.5858 92.15) (end 142.25 92.15) (width 0.6858) (layer F.Cu) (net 2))
 (segment (start 142.25 92.15) (end 140.9142 92.15) (width 0.6858) (layer F.Cu) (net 2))
 (segment (start 140.9142 92.15) (end 139.25 93.8142) (width 0.6858) (layer F.Cu) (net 2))
 (segment (start 139.25 93.8142) (end 139.25 98.75) (width 0.6858) (layer F.Cu) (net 2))
 (segment (start 155.5 76.75) (end 156 77.25) (width 0.6858) (layer F.Cu) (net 2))
 (segment (start 156 77.25) (end 156 79.5) (width 0.6858) (layer F.Cu) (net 2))
 (segment (start 147.404178 76.75) (end 155.5 76.75) (width 0.6858) (layer F.Cu) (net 2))
 (segment (start 146 78.154178) (end 147.404178 76.75) (width 0.6858) (layer F.Cu) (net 2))
 (segment (start 146 79.5) (end 146 78.154178) (width 0.6858) (layer F.Cu) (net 2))
 (segment (start 131.5 86.5) (end 131.5 84.525) (width 0.6858) (layer F.Cu) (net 1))
 (segment (start 131.5 88.975) (end 131.5 86.5) (width 0.6858) (layer F.Cu) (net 1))
 (via (at 131.5 86.5) (size 0.6858) (drill 0.3302) (layers F.Cu B.Cu) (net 1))
 (via (at 131.5 77.025) (size 0.6858) (drill 0.3302) (layers F.Cu B.Cu) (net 1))
 (via (at 131.5 96.225) (size 0.6858) (drill 0.3302) (layers F.Cu B.Cu) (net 1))
 (via (at 159.1 74) (size 0.6858) (drill 0.3302) (layers F.Cu B.Cu) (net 1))
 (via (at 148 93.5) (size 0.6858) (drill 0.3302) (layers F.Cu B.Cu) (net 1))
 (segment (start 131.5 81.475) (end 131.5 77.025) (width 0.6858) (layer F.Cu) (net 1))
 (segment (start 131.5 84.525) (end 131.5 80.75) (width 0.6858) (layer F.Cu) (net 1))
 (segment (start 131.5 91.775) (end 131.5 88.975) (width 0.6858) (layer F.Cu) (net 1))
 (segment (start 131.5 96.225) (end 131.5 91.775) (width 0.6858) (layer F.Cu) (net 1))
 (via (at 146 93.5) (size 0.6858) (drill 0.3302) (layers F.Cu B.Cu) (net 1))
 (via (at 146 93.5) (size 0.6858) (drill 0.3302) (layers F.Cu B.Cu) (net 1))
 (segment (start 138.75 82.25) (end 138.7108 82.25) (width 0.6858) (layer F.Cu) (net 6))
 (segment (start 138.7108 82.25) (end 136.4358 84.525) (width 0.6858) (layer F.Cu) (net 6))
 (segment (start 136.4358 84.525) (end 135 84.525) (width 0.6858) (layer F.Cu) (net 6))
 (segment (start 148.015862 81.72385) (end 147.499101 82.240611) (width 0.6858) (layer F.Cu) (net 6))
 (segment (start 147.499101 82.25) (end 138.759389 82.25) (width 0.6858) (layer F.Cu) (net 6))
 (segment (start 138.759389 82.240611) (end 138.75 82.25) (width 0.6858) (layer F.Cu) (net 6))
 (segment (start 150 79.5) (end 150 79.765862) (width 0.6858) (layer F.Cu) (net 6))
 (segment (start 150 79.765862) (end 148.015862 81.75) (width 0.6858) (layer F.Cu) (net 6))
 (segment (start 135 88.975) (end 135 84.525) (width 0.6858) (layer F.Cu) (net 6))
 (segment (start 135 91.775) (end 136.4358 91.775) (width 0.6858) (layer F.Cu) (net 5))
 (segment (start 136.4358 91.775) (end 137 91.2108) (width 0.6858) (layer F.Cu) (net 5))
 (segment (start 137 91.2108) (end 137 86.25) (width 0.6858) (layer F.Cu) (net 5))
 (segment (start 137 86.25) (end 140 83.25) (width 0.6858) (layer F.Cu) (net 5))
 (segment (start 140 83.25) (end 148.515861 83.25) (width 0.6858) (layer F.Cu) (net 5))
 (segment (start 148.515861 83.25) (end 149.015862 82.749999) (width 0.6858) (layer F.Cu) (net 5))
 (segment (start 149.015862 82.75) (end 152 79.765862) (width 0.6858) (layer F.Cu) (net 5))
 (segment (start 152 79.765862) (end 152 79.5) (width 0.6858) (layer F.Cu) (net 5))
 (segment (start 135 96.225) (end 135 91.775) (width 0.6858) (layer F.Cu) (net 5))
 (segment (start 148 79.5) (end 148 79.765862) (width 0.6858) (layer F.Cu) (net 7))
 (segment (start 148 79.765862) (end 146.515862 81.25) (width 0.6858) (layer F.Cu) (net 7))
 (segment (start 146.515862 81.25) (end 144.25 81.25) (width 0.6858) (layer F.Cu) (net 7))
 (segment (start 144.25 81.25) (end 143 80) (width 0.6858) (layer F.Cu) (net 7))
 (segment (start 143 80) (end 143 78.75) (width 0.6858) (layer F.Cu) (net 7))
 (segment (start 143 78.75) (end 141.275 77.025) (width 0.6858) (layer F.Cu) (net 7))
 (segment (start 141.275 77.025) (end 135 77.025) (width 0.6858) (layer F.Cu) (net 7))
 (segment (start 135 77.025) (end 135 81.475) (width 0.6858) (layer F.Cu) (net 7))
 (segment (start 147.25 86.5) (end 147.25 76.8) (width 0.6858) (layer B.Cu) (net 13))
 (segment (start 147.25 76.8) (end 150.05 74) (width 0.6858) (layer B.Cu) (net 13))
 (segment (start 150.05 74) (end 150.15 74) (width 0.6858) (layer B.Cu) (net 13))
 (via (at 150.15 74) (size 0.6858) (drill 0.3302) (layers F.Cu B.Cu) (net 13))
 (segment (start 159.5 86.5) (end 159.5 89.6858) (width 0.6858) (layer B.Cu) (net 10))
 (segment (start 159.5 89.6858) (end 156 93.1858) (width 0.6858) (layer B.Cu) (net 10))
 (segment (start 156 93.1858) (end 156 93.5) (width 0.6858) (layer B.Cu) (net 10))
 (via (at 156 93.5) (size 0.6858) (drill 0.3302) (layers F.Cu B.Cu) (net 10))
 (segment (start 156.4 74) (end 152.85 74) (width 0.6858) (layer F.Cu) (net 4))
 (segment (start 158 79.5) (end 158 77) (width 0.6858) (layer F.Cu) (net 4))
 (segment (start 158 77) (end 156.5 75.5) (width 0.6858) (layer F.Cu) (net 4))
 (segment (start 156.5 75.5) (end 156.5 74.1) (width 0.6858) (layer F.Cu) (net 4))
 (segment (start 156.5 74.1) (end 156.4 74) (width 0.6858) (layer F.Cu) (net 4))
 (segment (start 145.2358 96.5) (end 149.742081 96.5) (width 0.6858) (layer F.Cu) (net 8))
 (segment (start 149.742081 96.5) (end 150.54 97.297919) (width 0.6858) (layer F.Cu) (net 8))
 (segment (start 150.54 97.297919) (end 150.54 98.5) (width 0.6858) (layer F.Cu) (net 8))
 (segment (start 142.25 94.85) (end 143.5858 94.85) (width 0.6858) (layer F.Cu) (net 8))
 (segment (start 143.5858 94.85) (end 145.2358 96.5) (width 0.6858) (layer F.Cu) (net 8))
 (segment (start 152 97.04) (end 152 96.5) (width 0.6858) (layer F.Cu) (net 8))
 (segment (start 152 96.5) (end 152 93.5) (width 0.6858) (layer F.Cu) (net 8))
 (segment (start 150.54 98.5) (end 152 97.04) (width 0.6858) (layer F.Cu) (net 8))
 (segment (start 152 95.065) (end 152 93.5) (width 0.635) (layer F.Cu) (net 8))
 (segment (start 160.62 98.5) (end 158 95.88) (width 0.635) (layer F.Cu) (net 11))
 (segment (start 158 95.88) (end 158 93.5) (width 0.635) (layer F.Cu) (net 11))
 (segment (start 160 95.615014) (end 160 93.5) (width 0.635) (layer F.Cu) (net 12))
 (segment (start 162.884986 98.5) (end 160 95.615014) (width 0.635) (layer F.Cu) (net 12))
 (segment (start 163.16 98.5) (end 162.884986 98.5) (width 0.635) (layer F.Cu) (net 12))
 (segment (start 160 79.5) (end 154 79.5) (width 0.6858) (layer B.Cu) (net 3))
 (via (at 160 79.5) (size 0.6858) (drill 0.3302) (layers F.Cu B.Cu) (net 3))
 (via (at 154 79.5) (size 0.6858) (drill 0.3302) (layers F.Cu B.Cu) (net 3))
 (segment (start 153.375 86.5) (end 153.375 89.6858) (width 0.6858) (layer B.Cu) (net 9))
 (segment (start 153.375 89.6858) (end 154 90.3108) (width 0.6858) (layer B.Cu) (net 9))
 (segment (start 154 90.3108) (end 154 93.5) (width 0.6858) (layer B.Cu) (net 9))
 (via (at 154 93.5) (size 0.6858) (drill 0.3302) (layers F.Cu B.Cu) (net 9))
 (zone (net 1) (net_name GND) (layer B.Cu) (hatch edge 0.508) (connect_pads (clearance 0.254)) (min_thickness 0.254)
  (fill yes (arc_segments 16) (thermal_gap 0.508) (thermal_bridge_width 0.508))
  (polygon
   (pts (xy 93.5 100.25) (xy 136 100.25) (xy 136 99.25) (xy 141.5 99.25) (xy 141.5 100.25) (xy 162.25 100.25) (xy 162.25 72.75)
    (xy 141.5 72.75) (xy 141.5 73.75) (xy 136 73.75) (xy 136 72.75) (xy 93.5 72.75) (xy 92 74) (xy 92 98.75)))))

